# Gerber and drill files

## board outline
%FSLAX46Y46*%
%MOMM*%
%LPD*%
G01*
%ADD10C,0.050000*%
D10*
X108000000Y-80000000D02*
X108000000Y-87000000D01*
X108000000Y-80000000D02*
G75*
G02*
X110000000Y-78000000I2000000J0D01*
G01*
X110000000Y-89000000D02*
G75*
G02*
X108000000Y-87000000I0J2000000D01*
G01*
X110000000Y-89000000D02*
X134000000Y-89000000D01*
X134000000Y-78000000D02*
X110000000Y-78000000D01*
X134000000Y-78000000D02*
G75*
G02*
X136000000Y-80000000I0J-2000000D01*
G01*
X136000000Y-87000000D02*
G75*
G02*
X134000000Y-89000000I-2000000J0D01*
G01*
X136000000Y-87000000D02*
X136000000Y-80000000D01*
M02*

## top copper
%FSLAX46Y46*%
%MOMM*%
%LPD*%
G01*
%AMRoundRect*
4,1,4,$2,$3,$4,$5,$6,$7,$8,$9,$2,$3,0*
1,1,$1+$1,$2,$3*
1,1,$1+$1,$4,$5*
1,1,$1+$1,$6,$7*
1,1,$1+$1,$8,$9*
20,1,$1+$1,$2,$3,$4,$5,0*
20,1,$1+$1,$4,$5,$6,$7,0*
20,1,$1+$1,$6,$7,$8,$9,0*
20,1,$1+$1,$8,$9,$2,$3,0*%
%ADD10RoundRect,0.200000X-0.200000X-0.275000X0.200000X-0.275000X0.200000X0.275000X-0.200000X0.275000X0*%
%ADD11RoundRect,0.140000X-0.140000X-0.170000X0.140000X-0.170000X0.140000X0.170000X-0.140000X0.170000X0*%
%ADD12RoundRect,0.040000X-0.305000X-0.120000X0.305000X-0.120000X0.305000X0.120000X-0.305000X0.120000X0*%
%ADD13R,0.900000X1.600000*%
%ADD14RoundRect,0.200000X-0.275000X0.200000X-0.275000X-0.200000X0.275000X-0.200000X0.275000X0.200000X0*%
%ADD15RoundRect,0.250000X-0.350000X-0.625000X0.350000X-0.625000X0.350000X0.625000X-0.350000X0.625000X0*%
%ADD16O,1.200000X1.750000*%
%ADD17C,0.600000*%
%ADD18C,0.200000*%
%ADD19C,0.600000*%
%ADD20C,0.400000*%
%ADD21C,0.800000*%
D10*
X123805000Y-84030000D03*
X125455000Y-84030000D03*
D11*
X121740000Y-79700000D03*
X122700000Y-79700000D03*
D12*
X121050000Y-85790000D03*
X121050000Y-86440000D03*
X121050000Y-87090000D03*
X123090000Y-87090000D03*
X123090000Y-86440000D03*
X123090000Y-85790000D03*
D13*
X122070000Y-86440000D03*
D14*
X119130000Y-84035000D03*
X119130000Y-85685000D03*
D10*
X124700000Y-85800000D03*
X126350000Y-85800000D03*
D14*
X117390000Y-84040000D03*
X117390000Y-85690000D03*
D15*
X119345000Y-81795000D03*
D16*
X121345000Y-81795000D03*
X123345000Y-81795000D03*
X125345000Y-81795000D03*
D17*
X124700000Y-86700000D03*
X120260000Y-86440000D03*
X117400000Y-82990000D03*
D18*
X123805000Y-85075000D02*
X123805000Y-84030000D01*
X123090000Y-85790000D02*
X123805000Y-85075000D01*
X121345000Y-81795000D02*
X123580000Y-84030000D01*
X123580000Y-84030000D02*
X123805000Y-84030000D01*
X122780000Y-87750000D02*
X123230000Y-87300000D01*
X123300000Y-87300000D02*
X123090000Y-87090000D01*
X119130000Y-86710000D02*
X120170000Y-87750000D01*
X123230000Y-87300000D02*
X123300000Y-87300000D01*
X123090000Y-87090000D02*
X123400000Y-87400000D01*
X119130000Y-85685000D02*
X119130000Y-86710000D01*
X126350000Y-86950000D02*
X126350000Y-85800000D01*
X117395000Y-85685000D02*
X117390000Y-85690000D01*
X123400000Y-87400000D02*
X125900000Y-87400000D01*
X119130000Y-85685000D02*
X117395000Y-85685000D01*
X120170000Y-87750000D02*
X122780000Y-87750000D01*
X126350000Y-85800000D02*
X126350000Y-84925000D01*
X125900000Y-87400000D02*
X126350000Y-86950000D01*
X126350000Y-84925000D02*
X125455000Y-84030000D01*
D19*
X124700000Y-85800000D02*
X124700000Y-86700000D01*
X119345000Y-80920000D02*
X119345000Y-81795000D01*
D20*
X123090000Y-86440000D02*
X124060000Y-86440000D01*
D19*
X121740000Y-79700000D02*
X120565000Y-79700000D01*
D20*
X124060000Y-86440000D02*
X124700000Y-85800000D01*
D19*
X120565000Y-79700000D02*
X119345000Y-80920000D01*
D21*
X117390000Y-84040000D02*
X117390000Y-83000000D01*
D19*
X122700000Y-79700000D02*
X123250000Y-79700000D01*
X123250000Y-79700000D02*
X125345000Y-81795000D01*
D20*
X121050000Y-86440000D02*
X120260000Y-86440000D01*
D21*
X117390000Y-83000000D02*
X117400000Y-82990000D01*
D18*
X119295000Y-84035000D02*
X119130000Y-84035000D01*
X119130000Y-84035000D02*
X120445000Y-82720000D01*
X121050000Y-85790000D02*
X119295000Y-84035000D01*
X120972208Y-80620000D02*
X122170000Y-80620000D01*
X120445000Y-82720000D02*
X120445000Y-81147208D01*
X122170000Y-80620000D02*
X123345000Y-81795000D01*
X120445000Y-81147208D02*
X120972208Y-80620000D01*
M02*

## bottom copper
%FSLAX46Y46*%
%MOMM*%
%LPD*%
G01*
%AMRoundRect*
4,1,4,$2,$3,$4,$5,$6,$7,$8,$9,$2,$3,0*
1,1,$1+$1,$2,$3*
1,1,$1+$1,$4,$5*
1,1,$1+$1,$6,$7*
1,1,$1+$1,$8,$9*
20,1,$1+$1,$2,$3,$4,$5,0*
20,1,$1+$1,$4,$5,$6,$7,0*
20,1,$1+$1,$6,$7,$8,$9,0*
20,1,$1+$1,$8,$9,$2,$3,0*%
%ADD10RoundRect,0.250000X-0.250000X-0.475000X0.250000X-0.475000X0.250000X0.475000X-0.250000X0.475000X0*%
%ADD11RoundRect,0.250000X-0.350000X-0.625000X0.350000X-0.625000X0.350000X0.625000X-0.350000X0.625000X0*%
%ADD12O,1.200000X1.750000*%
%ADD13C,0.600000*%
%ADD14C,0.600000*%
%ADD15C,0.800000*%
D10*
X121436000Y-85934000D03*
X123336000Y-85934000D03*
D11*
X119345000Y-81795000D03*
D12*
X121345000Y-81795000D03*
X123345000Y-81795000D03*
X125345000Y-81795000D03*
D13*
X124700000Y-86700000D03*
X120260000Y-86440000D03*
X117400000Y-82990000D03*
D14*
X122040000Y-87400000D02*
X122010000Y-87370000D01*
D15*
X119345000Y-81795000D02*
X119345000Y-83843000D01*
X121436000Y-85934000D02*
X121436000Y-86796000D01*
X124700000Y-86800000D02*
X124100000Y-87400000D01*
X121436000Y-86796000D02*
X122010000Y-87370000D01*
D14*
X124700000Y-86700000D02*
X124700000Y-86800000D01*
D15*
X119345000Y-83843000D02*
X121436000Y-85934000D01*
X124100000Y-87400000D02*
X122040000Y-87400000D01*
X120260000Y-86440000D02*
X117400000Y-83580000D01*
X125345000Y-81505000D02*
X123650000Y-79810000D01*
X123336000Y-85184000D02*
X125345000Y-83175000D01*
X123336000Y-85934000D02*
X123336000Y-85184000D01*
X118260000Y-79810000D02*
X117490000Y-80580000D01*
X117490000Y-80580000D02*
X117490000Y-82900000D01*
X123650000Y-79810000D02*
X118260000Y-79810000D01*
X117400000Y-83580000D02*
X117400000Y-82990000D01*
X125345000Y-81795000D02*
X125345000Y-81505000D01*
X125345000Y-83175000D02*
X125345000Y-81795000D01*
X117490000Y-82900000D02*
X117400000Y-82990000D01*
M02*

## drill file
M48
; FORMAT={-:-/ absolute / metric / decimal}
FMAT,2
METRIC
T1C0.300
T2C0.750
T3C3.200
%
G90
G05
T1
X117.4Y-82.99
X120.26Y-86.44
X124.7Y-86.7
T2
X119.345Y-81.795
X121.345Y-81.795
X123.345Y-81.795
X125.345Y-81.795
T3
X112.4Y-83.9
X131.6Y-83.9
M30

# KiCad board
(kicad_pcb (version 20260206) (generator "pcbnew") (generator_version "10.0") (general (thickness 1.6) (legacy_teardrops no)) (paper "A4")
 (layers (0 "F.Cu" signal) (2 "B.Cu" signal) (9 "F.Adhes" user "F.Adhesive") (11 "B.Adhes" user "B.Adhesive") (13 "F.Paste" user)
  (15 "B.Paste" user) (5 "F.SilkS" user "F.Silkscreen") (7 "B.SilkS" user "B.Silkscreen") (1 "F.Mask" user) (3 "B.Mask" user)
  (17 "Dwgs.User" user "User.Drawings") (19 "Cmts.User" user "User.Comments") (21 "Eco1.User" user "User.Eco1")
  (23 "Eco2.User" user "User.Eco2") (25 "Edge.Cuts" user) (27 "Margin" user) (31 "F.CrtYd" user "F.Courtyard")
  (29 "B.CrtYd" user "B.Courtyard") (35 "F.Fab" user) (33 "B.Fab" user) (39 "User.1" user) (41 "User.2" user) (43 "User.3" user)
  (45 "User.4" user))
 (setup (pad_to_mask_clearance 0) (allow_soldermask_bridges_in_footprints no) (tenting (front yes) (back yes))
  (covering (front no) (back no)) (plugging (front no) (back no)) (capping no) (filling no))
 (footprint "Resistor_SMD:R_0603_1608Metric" (layer "F.Cu") (at 124.63 84.03)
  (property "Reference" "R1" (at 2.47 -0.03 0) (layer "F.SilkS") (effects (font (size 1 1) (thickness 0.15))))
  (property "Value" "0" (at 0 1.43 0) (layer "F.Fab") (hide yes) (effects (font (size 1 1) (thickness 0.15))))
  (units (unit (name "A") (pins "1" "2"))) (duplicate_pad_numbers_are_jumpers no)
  (pad "1" smd roundrect (at -0.825 0) (size 0.8 0.95) (layers "F.Cu" "F.Mask" "F.Paste") (roundrect_rratio 0.25) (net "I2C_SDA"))
  (pad "2" smd roundrect (at 0.825 0) (size 0.8 0.95) (layers "F.Cu" "F.Mask" "F.Paste") (roundrect_rratio 0.25) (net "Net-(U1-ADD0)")))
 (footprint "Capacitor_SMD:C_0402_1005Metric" (layer "F.Cu") (at 122.22 79.7)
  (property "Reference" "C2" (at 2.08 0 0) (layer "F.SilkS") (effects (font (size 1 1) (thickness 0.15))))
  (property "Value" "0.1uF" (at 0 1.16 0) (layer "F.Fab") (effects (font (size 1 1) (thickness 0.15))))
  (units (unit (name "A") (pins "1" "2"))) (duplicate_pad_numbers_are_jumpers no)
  (pad "1" smd roundrect (at -0.48 0) (size 0.56 0.62) (layers "F.Cu" "F.Mask" "F.Paste") (roundrect_rratio 0.25) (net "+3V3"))
  (pad "2" smd roundrect (at 0.48 0) (size 0.56 0.62) (layers "F.Cu" "F.Mask" "F.Paste") (roundrect_rratio 0.25) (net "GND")))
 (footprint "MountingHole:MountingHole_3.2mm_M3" (layer "F.Cu") (at 112.4 83.9)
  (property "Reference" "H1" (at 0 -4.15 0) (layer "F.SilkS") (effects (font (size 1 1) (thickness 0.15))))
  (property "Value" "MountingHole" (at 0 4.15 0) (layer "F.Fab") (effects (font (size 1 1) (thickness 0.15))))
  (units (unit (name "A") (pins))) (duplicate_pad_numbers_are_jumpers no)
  (pad "" np_thru_hole circle (at 0 0) (size 3.2 3.2) (drill 3.2) (layers "*.Cu" "*.Mask")))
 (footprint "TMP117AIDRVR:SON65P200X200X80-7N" (layer "F.Cu") (at 122.07 86.44)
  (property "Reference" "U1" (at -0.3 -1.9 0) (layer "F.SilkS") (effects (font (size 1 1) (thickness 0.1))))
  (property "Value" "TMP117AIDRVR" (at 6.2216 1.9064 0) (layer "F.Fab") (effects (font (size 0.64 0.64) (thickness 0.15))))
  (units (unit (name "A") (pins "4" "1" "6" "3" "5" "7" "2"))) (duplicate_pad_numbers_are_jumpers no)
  (pad "1" smd roundrect (at -1.02 -0.65) (size 0.69 0.32) (layers "F.Cu" "F.Mask" "F.Paste") (roundrect_rratio 0.125) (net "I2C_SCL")
   (solder_mask_margin 0))
  (pad "2" smd roundrect (at -1.02 0) (size 0.69 0.32) (layers "F.Cu" "F.Mask" "F.Paste") (roundrect_rratio 0.125) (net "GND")
   (solder_mask_margin 0))
  (pad "3" smd roundrect (at -1.02 0.65) (size 0.69 0.32) (layers "F.Cu" "F.Mask" "F.Paste") (roundrect_rratio 0.125)
   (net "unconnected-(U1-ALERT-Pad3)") (solder_mask_margin 0))
  (pad "4" smd roundrect (at 1.02 0.65) (size 0.69 0.32) (layers "F.Cu" "F.Mask" "F.Paste") (roundrect_rratio 0.125) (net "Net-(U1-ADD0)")
   (solder_mask_margin 0))
  (pad "5" smd roundrect (at 1.02 0) (size 0.69 0.32) (layers "F.Cu" "F.Mask" "F.Paste") (roundrect_rratio 0.125) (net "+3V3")
   (solder_mask_margin 0))
  (pad "6" smd roundrect (at 1.02 -0.65) (size 0.69 0.32) (layers "F.Cu" "F.Mask" "F.Paste") (roundrect_rratio 0.125) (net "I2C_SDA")
   (solder_mask_margin 0))
  (pad "7" smd rect (at 0 0) (size 0.9 1.6) (layers "F.Cu") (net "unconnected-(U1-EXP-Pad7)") (solder_mask_margin 0.102)))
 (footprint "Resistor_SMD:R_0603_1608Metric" (layer "F.Cu") (at 119.13 84.86 -90)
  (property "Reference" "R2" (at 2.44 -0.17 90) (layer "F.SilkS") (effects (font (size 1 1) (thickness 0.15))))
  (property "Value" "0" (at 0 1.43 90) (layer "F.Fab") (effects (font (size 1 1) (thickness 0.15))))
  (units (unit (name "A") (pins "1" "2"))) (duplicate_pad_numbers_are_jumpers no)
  (pad "1" smd roundrect (at -0.825 0 270) (size 0.8 0.95) (layers "F.Cu" "F.Mask" "F.Paste") (roundrect_rratio 0.25) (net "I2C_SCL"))
  (pad "2" smd roundrect (at 0.825 0 270) (size 0.8 0.95) (layers "F.Cu" "F.Mask" "F.Paste") (roundrect_rratio 0.25) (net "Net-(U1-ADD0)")))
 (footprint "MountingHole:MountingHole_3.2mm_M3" (layer "F.Cu") (at 131.6 83.9)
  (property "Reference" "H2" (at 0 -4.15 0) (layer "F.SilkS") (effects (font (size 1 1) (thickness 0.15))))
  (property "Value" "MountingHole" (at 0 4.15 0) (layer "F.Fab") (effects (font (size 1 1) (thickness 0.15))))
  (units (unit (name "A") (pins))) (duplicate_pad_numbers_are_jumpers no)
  (pad "" np_thru_hole circle (at 0 0) (size 3.2 3.2) (drill 3.2) (layers "*.Cu" "*.Mask")))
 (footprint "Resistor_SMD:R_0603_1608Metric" (layer "F.Cu") (at 125.525 85.8)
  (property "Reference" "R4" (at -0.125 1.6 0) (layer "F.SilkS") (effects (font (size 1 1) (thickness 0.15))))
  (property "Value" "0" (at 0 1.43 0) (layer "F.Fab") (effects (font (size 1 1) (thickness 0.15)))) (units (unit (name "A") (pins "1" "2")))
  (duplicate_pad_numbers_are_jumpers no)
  (pad "1" smd roundrect (at -0.825 0) (size 0.8 0.95) (layers "F.Cu" "F.Mask" "F.Paste") (roundrect_rratio 0.25) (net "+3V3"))
  (pad "2" smd roundrect (at 0.825 0) (size 0.8 0.95) (layers "F.Cu" "F.Mask" "F.Paste") (roundrect_rratio 0.25) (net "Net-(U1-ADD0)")))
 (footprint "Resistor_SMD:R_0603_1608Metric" (layer "F.Cu") (at 117.39 84.865 -90)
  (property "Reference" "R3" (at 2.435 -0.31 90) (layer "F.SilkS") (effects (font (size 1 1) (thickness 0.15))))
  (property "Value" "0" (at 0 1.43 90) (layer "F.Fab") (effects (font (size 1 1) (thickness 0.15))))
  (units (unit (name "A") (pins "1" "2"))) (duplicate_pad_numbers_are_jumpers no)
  (pad "1" smd roundrect (at -0.825 0 270) (size 0.8 0.95) (layers "F.Cu" "F.Mask" "F.Paste") (roundrect_rratio 0.25) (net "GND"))
  (pad "2" smd roundrect (at 0.825 0 270) (size 0.8 0.95) (layers "F.Cu" "F.Mask" "F.Paste") (roundrect_rratio 0.25) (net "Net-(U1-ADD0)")))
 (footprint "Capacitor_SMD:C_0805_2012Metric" (layer "B.Cu") (at 122.386 85.934)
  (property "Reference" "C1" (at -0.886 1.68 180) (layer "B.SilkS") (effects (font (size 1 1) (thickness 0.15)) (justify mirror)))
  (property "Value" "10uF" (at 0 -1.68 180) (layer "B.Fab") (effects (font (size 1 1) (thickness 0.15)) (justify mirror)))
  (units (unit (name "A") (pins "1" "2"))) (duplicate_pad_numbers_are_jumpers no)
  (pad "1" smd roundrect (at -0.95 0) (size 1 1.45) (layers "B.Cu" "B.Mask" "B.Paste") (roundrect_rratio 0.25) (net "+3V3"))
  (pad "2" smd roundrect (at 0.95 0) (size 1 1.45) (layers "B.Cu" "B.Mask" "B.Paste") (roundrect_rratio 0.25) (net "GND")))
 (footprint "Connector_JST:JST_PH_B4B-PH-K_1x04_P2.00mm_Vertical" (layer "B.Cu") (at 119.345 81.795)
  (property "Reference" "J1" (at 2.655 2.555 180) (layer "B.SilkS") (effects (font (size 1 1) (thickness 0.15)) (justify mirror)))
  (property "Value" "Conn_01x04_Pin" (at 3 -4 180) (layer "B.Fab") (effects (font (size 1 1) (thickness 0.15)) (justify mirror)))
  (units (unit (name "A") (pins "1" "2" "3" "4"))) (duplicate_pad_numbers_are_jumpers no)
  (pad "1" thru_hole roundrect (at 0 0) (size 1.2 1.75) (drill 0.75) (layers "*.Cu" "*.Mask") (remove_unused_layers no)
   (roundrect_rratio 0.208333) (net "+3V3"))
  (pad "2" thru_hole oval (at 2 0) (size 1.2 1.75) (drill 0.75) (layers "*.Cu" "*.Mask") (remove_unused_layers no) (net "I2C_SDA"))
  (pad "3" thru_hole oval (at 4 0) (size 1.2 1.75) (drill 0.75) (layers "*.Cu" "*.Mask") (remove_unused_layers no) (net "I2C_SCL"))
  (pad "4" thru_hole oval (at 6 0) (size 1.2 1.75) (drill 0.75) (layers "*.Cu" "*.Mask") (remove_unused_layers no) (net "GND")))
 (gr_line (start 108 80) (end 108 87) (stroke (width 0.05) (type default)) (layer "Edge.Cuts"))
 (gr_arc (start 108 80) (mid 108.585786 78.585786) (end 110 78) (stroke (width 0.05) (type default)) (layer "Edge.Cuts"))
 (gr_arc (start 110 89) (mid 108.585786 88.414214) (end 108 87) (stroke (width 0.05) (type default)) (layer "Edge.Cuts"))
 (gr_line (start 110 89) (end 134 89) (stroke (width 0.05) (type default)) (layer "Edge.Cuts"))
 (gr_line (start 134 78) (end 110 78) (stroke (width 0.05) (type default)) (layer "Edge.Cuts"))
 (gr_arc (start 134 78) (mid 135.414214 78.585786) (end 136 80) (stroke (width 0.05) (type default)) (layer "Edge.Cuts"))
 (gr_arc (start 136 87) (mid 135.414214 88.414214) (end 134 89) (stroke (width 0.05) (type default)) (layer "Edge.Cuts"))
 (gr_line (start 136 87) (end 136 80) (stroke (width 0.05) (type default)) (layer "Edge.Cuts"))
 (segment (start 123.805 85.075) (end 123.805 84.03) (width 0.2) (layer "F.Cu") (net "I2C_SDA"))
 (segment (start 123.09 85.79) (end 123.805 85.075) (width 0.2) (layer "F.Cu") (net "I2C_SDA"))
 (segment (start 121.345 81.795) (end 123.58 84.03) (width 0.2) (layer "F.Cu") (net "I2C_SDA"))
 (segment (start 123.58 84.03) (end 123.805 84.03) (width 0.2) (layer "F.Cu") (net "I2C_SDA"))
 (segment (start 122.78 87.75) (end 123.23 87.3) (width 0.2) (layer "F.Cu") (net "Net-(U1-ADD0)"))
 (segment (start 123.3 87.3) (end 123.09 87.09) (width 0.2) (layer "F.Cu") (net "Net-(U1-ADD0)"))
 (segment (start 119.13 86.71) (end 120.17 87.75) (width 0.2) (layer "F.Cu") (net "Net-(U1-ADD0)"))
 (segment (start 123.23 87.3) (end 123.3 87.3) (width 0.2) (layer "F.Cu") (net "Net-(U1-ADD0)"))
 (segment (start 123.09 87.09) (end 123.4 87.4) (width 0.2) (layer "F.Cu") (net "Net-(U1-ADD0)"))
 (segment (start 119.13 85.685) (end 119.13 86.71) (width 0.2) (layer "F.Cu") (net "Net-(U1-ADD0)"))
 (segment (start 126.35 86.95) (end 126.35 85.8) (width 0.2) (layer "F.Cu") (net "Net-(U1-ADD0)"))
 (segment (start 117.395 85.685) (end 117.39 85.69) (width 0.2) (layer "F.Cu") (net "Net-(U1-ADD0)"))
 (segment (start 123.4 87.4) (end 125.9 87.4) (width 0.2) (layer "F.Cu") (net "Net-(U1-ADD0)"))
 (segment (start 119.13 85.685) (end 117.395 85.685) (width 0.2) (layer "F.Cu") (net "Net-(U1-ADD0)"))
 (segment (start 120.17 87.75) (end 122.78 87.75) (width 0.2) (layer "F.Cu") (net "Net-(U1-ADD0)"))
 (segment (start 126.35 85.8) (end 126.35 84.925) (width 0.2) (layer "F.Cu") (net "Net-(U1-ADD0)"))
 (segment (start 125.9 87.4) (end 126.35 86.95) (width 0.2) (layer "F.Cu") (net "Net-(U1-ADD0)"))
 (segment (start 126.35 84.925) (end 125.455 84.03) (width 0.2) (layer "F.Cu") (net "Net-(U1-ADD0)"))
 (segment (start 124.7 85.8) (end 124.7 86.7) (width 0.6) (layer "F.Cu") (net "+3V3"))
 (segment (start 119.345 80.92) (end 119.345 81.795) (width 0.6) (layer "F.Cu") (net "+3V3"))
 (segment (start 123.09 86.44) (end 124.06 86.44) (width 0.4) (layer "F.Cu") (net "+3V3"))
 (segment (start 121.74 79.7) (end 120.565 79.7) (width 0.6) (layer "F.Cu") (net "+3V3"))
 (segment (start 124.06 86.44) (end 124.7 85.8) (width 0.4) (layer "F.Cu") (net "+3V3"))
 (segment (start 120.565 79.7) (end 119.345 80.92) (width 0.6) (layer "F.Cu") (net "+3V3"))
 (via (at 124.7 86.7) (size 0.6) (drill 0.3) (layers "F.Cu" "B.Cu") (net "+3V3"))
 (segment (start 122.04 87.4) (end 122.01 87.37) (width 0.6) (layer "B.Cu") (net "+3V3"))
 (segment (start 119.345 81.795) (end 119.345 83.843) (width 0.8) (layer "B.Cu") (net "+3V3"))
 (segment (start 121.436 85.934) (end 121.436 86.796) (width 0.8) (layer "B.Cu") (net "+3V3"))
 (segment (start 124.7 86.8) (end 124.1 87.4) (width 0.8) (layer "B.Cu") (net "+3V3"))
 (segment (start 121.436 86.796) (end 122.01 87.37) (width 0.8) (layer "B.Cu") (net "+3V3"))
 (segment (start 124.7 86.7) (end 124.7 86.8) (width 0.6) (layer "B.Cu") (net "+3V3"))
 (segment (start 119.345 83.843) (end 121.436 85.934) (width 0.8) (layer "B.Cu") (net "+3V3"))
 (segment (start 124.1 87.4) (end 122.04 87.4) (width 0.8) (layer "B.Cu") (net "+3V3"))
 (segment (start 117.39 84.04) (end 117.39 83) (width 0.8) (layer "F.Cu") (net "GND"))
 (segment (start 122.7 79.7) (end 123.25 79.7) (width 0.6) (layer "F.Cu") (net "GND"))
 (segment (start 123.25 79.7) (end 125.345 81.795) (width 0.6) (layer "F.Cu") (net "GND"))
 (segment (start 121.05 86.44) (end 120.26 86.44) (width 0.4) (layer "F.Cu") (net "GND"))
 (segment (start 117.39 83) (end 117.4 82.99) (width 0.8) (layer "F.Cu") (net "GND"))
 (via (at 120.26 86.44) (size 0.6) (drill 0.3) (layers "F.Cu" "B.Cu") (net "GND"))
 (via (at 117.4 82.99) (size 0.6) (drill 0.3) (layers "F.Cu" "B.Cu") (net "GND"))
 (segment (start 120.26 86.44) (end 117.4 83.58) (width 0.8) (layer "B.Cu") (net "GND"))
 (segment (start 125.345 81.505) (end 123.65 79.81) (width 0.8) (layer "B.Cu") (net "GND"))
 (segment (start 123.336 85.184) (end 125.345 83.175) (width 0.8) (layer "B.Cu") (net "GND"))
 (segment (start 123.336 85.934) (end 123.336 85.184) (width 0.8) (layer "B.Cu") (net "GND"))
 (segment (start 118.26 79.81) (end 117.49 80.58) (width 0.8) (layer "B.Cu") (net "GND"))
 (segment (start 117.49 80.58) (end 117.49 82.9) (width 0.8) (layer "B.Cu") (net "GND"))
 (segment (start 123.65 79.81) (end 118.26 79.81) (width 0.8) (layer "B.Cu") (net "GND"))
 (segment (start 117.4 83.58) (end 117.4 82.99) (width 0.8) (layer "B.Cu") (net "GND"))
 (segment (start 125.345 81.795) (end 125.345 81.505) (width 0.8) (layer "B.Cu") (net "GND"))
 (segment (start 125.345 83.175) (end 125.345 81.795) (width 0.8) (layer "B.Cu") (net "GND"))
 (segment (start 117.49 82.9) (end 117.4 82.99) (width 0.8) (layer "B.Cu") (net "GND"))
 (segment (start 119.295 84.035) (end 119.13 84.035) (width 0.2) (layer "F.Cu") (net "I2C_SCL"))
 (segment (start 119.13 84.035) (end 120.445 82.72) (width 0.2) (layer "F.Cu") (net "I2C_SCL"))
 (segment (start 121.05 85.79) (end 119.295 84.035) (width 0.2) (layer "F.Cu") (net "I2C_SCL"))
 (segment (start 120.972208 80.62) (end 122.17 80.62) (width 0.2) (layer "F.Cu") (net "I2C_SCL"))
 (segment (start 120.445 82.72) (end 120.445 81.147208) (width 0.2) (layer "F.Cu") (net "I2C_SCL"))
 (segment (start 122.17 80.62) (end 123.345 81.795) (width 0.2) (layer "F.Cu") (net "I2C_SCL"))
 (segment (start 120.445 81.147208) (end 120.972208 80.62) (width 0.2) (layer "F.Cu") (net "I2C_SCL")))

